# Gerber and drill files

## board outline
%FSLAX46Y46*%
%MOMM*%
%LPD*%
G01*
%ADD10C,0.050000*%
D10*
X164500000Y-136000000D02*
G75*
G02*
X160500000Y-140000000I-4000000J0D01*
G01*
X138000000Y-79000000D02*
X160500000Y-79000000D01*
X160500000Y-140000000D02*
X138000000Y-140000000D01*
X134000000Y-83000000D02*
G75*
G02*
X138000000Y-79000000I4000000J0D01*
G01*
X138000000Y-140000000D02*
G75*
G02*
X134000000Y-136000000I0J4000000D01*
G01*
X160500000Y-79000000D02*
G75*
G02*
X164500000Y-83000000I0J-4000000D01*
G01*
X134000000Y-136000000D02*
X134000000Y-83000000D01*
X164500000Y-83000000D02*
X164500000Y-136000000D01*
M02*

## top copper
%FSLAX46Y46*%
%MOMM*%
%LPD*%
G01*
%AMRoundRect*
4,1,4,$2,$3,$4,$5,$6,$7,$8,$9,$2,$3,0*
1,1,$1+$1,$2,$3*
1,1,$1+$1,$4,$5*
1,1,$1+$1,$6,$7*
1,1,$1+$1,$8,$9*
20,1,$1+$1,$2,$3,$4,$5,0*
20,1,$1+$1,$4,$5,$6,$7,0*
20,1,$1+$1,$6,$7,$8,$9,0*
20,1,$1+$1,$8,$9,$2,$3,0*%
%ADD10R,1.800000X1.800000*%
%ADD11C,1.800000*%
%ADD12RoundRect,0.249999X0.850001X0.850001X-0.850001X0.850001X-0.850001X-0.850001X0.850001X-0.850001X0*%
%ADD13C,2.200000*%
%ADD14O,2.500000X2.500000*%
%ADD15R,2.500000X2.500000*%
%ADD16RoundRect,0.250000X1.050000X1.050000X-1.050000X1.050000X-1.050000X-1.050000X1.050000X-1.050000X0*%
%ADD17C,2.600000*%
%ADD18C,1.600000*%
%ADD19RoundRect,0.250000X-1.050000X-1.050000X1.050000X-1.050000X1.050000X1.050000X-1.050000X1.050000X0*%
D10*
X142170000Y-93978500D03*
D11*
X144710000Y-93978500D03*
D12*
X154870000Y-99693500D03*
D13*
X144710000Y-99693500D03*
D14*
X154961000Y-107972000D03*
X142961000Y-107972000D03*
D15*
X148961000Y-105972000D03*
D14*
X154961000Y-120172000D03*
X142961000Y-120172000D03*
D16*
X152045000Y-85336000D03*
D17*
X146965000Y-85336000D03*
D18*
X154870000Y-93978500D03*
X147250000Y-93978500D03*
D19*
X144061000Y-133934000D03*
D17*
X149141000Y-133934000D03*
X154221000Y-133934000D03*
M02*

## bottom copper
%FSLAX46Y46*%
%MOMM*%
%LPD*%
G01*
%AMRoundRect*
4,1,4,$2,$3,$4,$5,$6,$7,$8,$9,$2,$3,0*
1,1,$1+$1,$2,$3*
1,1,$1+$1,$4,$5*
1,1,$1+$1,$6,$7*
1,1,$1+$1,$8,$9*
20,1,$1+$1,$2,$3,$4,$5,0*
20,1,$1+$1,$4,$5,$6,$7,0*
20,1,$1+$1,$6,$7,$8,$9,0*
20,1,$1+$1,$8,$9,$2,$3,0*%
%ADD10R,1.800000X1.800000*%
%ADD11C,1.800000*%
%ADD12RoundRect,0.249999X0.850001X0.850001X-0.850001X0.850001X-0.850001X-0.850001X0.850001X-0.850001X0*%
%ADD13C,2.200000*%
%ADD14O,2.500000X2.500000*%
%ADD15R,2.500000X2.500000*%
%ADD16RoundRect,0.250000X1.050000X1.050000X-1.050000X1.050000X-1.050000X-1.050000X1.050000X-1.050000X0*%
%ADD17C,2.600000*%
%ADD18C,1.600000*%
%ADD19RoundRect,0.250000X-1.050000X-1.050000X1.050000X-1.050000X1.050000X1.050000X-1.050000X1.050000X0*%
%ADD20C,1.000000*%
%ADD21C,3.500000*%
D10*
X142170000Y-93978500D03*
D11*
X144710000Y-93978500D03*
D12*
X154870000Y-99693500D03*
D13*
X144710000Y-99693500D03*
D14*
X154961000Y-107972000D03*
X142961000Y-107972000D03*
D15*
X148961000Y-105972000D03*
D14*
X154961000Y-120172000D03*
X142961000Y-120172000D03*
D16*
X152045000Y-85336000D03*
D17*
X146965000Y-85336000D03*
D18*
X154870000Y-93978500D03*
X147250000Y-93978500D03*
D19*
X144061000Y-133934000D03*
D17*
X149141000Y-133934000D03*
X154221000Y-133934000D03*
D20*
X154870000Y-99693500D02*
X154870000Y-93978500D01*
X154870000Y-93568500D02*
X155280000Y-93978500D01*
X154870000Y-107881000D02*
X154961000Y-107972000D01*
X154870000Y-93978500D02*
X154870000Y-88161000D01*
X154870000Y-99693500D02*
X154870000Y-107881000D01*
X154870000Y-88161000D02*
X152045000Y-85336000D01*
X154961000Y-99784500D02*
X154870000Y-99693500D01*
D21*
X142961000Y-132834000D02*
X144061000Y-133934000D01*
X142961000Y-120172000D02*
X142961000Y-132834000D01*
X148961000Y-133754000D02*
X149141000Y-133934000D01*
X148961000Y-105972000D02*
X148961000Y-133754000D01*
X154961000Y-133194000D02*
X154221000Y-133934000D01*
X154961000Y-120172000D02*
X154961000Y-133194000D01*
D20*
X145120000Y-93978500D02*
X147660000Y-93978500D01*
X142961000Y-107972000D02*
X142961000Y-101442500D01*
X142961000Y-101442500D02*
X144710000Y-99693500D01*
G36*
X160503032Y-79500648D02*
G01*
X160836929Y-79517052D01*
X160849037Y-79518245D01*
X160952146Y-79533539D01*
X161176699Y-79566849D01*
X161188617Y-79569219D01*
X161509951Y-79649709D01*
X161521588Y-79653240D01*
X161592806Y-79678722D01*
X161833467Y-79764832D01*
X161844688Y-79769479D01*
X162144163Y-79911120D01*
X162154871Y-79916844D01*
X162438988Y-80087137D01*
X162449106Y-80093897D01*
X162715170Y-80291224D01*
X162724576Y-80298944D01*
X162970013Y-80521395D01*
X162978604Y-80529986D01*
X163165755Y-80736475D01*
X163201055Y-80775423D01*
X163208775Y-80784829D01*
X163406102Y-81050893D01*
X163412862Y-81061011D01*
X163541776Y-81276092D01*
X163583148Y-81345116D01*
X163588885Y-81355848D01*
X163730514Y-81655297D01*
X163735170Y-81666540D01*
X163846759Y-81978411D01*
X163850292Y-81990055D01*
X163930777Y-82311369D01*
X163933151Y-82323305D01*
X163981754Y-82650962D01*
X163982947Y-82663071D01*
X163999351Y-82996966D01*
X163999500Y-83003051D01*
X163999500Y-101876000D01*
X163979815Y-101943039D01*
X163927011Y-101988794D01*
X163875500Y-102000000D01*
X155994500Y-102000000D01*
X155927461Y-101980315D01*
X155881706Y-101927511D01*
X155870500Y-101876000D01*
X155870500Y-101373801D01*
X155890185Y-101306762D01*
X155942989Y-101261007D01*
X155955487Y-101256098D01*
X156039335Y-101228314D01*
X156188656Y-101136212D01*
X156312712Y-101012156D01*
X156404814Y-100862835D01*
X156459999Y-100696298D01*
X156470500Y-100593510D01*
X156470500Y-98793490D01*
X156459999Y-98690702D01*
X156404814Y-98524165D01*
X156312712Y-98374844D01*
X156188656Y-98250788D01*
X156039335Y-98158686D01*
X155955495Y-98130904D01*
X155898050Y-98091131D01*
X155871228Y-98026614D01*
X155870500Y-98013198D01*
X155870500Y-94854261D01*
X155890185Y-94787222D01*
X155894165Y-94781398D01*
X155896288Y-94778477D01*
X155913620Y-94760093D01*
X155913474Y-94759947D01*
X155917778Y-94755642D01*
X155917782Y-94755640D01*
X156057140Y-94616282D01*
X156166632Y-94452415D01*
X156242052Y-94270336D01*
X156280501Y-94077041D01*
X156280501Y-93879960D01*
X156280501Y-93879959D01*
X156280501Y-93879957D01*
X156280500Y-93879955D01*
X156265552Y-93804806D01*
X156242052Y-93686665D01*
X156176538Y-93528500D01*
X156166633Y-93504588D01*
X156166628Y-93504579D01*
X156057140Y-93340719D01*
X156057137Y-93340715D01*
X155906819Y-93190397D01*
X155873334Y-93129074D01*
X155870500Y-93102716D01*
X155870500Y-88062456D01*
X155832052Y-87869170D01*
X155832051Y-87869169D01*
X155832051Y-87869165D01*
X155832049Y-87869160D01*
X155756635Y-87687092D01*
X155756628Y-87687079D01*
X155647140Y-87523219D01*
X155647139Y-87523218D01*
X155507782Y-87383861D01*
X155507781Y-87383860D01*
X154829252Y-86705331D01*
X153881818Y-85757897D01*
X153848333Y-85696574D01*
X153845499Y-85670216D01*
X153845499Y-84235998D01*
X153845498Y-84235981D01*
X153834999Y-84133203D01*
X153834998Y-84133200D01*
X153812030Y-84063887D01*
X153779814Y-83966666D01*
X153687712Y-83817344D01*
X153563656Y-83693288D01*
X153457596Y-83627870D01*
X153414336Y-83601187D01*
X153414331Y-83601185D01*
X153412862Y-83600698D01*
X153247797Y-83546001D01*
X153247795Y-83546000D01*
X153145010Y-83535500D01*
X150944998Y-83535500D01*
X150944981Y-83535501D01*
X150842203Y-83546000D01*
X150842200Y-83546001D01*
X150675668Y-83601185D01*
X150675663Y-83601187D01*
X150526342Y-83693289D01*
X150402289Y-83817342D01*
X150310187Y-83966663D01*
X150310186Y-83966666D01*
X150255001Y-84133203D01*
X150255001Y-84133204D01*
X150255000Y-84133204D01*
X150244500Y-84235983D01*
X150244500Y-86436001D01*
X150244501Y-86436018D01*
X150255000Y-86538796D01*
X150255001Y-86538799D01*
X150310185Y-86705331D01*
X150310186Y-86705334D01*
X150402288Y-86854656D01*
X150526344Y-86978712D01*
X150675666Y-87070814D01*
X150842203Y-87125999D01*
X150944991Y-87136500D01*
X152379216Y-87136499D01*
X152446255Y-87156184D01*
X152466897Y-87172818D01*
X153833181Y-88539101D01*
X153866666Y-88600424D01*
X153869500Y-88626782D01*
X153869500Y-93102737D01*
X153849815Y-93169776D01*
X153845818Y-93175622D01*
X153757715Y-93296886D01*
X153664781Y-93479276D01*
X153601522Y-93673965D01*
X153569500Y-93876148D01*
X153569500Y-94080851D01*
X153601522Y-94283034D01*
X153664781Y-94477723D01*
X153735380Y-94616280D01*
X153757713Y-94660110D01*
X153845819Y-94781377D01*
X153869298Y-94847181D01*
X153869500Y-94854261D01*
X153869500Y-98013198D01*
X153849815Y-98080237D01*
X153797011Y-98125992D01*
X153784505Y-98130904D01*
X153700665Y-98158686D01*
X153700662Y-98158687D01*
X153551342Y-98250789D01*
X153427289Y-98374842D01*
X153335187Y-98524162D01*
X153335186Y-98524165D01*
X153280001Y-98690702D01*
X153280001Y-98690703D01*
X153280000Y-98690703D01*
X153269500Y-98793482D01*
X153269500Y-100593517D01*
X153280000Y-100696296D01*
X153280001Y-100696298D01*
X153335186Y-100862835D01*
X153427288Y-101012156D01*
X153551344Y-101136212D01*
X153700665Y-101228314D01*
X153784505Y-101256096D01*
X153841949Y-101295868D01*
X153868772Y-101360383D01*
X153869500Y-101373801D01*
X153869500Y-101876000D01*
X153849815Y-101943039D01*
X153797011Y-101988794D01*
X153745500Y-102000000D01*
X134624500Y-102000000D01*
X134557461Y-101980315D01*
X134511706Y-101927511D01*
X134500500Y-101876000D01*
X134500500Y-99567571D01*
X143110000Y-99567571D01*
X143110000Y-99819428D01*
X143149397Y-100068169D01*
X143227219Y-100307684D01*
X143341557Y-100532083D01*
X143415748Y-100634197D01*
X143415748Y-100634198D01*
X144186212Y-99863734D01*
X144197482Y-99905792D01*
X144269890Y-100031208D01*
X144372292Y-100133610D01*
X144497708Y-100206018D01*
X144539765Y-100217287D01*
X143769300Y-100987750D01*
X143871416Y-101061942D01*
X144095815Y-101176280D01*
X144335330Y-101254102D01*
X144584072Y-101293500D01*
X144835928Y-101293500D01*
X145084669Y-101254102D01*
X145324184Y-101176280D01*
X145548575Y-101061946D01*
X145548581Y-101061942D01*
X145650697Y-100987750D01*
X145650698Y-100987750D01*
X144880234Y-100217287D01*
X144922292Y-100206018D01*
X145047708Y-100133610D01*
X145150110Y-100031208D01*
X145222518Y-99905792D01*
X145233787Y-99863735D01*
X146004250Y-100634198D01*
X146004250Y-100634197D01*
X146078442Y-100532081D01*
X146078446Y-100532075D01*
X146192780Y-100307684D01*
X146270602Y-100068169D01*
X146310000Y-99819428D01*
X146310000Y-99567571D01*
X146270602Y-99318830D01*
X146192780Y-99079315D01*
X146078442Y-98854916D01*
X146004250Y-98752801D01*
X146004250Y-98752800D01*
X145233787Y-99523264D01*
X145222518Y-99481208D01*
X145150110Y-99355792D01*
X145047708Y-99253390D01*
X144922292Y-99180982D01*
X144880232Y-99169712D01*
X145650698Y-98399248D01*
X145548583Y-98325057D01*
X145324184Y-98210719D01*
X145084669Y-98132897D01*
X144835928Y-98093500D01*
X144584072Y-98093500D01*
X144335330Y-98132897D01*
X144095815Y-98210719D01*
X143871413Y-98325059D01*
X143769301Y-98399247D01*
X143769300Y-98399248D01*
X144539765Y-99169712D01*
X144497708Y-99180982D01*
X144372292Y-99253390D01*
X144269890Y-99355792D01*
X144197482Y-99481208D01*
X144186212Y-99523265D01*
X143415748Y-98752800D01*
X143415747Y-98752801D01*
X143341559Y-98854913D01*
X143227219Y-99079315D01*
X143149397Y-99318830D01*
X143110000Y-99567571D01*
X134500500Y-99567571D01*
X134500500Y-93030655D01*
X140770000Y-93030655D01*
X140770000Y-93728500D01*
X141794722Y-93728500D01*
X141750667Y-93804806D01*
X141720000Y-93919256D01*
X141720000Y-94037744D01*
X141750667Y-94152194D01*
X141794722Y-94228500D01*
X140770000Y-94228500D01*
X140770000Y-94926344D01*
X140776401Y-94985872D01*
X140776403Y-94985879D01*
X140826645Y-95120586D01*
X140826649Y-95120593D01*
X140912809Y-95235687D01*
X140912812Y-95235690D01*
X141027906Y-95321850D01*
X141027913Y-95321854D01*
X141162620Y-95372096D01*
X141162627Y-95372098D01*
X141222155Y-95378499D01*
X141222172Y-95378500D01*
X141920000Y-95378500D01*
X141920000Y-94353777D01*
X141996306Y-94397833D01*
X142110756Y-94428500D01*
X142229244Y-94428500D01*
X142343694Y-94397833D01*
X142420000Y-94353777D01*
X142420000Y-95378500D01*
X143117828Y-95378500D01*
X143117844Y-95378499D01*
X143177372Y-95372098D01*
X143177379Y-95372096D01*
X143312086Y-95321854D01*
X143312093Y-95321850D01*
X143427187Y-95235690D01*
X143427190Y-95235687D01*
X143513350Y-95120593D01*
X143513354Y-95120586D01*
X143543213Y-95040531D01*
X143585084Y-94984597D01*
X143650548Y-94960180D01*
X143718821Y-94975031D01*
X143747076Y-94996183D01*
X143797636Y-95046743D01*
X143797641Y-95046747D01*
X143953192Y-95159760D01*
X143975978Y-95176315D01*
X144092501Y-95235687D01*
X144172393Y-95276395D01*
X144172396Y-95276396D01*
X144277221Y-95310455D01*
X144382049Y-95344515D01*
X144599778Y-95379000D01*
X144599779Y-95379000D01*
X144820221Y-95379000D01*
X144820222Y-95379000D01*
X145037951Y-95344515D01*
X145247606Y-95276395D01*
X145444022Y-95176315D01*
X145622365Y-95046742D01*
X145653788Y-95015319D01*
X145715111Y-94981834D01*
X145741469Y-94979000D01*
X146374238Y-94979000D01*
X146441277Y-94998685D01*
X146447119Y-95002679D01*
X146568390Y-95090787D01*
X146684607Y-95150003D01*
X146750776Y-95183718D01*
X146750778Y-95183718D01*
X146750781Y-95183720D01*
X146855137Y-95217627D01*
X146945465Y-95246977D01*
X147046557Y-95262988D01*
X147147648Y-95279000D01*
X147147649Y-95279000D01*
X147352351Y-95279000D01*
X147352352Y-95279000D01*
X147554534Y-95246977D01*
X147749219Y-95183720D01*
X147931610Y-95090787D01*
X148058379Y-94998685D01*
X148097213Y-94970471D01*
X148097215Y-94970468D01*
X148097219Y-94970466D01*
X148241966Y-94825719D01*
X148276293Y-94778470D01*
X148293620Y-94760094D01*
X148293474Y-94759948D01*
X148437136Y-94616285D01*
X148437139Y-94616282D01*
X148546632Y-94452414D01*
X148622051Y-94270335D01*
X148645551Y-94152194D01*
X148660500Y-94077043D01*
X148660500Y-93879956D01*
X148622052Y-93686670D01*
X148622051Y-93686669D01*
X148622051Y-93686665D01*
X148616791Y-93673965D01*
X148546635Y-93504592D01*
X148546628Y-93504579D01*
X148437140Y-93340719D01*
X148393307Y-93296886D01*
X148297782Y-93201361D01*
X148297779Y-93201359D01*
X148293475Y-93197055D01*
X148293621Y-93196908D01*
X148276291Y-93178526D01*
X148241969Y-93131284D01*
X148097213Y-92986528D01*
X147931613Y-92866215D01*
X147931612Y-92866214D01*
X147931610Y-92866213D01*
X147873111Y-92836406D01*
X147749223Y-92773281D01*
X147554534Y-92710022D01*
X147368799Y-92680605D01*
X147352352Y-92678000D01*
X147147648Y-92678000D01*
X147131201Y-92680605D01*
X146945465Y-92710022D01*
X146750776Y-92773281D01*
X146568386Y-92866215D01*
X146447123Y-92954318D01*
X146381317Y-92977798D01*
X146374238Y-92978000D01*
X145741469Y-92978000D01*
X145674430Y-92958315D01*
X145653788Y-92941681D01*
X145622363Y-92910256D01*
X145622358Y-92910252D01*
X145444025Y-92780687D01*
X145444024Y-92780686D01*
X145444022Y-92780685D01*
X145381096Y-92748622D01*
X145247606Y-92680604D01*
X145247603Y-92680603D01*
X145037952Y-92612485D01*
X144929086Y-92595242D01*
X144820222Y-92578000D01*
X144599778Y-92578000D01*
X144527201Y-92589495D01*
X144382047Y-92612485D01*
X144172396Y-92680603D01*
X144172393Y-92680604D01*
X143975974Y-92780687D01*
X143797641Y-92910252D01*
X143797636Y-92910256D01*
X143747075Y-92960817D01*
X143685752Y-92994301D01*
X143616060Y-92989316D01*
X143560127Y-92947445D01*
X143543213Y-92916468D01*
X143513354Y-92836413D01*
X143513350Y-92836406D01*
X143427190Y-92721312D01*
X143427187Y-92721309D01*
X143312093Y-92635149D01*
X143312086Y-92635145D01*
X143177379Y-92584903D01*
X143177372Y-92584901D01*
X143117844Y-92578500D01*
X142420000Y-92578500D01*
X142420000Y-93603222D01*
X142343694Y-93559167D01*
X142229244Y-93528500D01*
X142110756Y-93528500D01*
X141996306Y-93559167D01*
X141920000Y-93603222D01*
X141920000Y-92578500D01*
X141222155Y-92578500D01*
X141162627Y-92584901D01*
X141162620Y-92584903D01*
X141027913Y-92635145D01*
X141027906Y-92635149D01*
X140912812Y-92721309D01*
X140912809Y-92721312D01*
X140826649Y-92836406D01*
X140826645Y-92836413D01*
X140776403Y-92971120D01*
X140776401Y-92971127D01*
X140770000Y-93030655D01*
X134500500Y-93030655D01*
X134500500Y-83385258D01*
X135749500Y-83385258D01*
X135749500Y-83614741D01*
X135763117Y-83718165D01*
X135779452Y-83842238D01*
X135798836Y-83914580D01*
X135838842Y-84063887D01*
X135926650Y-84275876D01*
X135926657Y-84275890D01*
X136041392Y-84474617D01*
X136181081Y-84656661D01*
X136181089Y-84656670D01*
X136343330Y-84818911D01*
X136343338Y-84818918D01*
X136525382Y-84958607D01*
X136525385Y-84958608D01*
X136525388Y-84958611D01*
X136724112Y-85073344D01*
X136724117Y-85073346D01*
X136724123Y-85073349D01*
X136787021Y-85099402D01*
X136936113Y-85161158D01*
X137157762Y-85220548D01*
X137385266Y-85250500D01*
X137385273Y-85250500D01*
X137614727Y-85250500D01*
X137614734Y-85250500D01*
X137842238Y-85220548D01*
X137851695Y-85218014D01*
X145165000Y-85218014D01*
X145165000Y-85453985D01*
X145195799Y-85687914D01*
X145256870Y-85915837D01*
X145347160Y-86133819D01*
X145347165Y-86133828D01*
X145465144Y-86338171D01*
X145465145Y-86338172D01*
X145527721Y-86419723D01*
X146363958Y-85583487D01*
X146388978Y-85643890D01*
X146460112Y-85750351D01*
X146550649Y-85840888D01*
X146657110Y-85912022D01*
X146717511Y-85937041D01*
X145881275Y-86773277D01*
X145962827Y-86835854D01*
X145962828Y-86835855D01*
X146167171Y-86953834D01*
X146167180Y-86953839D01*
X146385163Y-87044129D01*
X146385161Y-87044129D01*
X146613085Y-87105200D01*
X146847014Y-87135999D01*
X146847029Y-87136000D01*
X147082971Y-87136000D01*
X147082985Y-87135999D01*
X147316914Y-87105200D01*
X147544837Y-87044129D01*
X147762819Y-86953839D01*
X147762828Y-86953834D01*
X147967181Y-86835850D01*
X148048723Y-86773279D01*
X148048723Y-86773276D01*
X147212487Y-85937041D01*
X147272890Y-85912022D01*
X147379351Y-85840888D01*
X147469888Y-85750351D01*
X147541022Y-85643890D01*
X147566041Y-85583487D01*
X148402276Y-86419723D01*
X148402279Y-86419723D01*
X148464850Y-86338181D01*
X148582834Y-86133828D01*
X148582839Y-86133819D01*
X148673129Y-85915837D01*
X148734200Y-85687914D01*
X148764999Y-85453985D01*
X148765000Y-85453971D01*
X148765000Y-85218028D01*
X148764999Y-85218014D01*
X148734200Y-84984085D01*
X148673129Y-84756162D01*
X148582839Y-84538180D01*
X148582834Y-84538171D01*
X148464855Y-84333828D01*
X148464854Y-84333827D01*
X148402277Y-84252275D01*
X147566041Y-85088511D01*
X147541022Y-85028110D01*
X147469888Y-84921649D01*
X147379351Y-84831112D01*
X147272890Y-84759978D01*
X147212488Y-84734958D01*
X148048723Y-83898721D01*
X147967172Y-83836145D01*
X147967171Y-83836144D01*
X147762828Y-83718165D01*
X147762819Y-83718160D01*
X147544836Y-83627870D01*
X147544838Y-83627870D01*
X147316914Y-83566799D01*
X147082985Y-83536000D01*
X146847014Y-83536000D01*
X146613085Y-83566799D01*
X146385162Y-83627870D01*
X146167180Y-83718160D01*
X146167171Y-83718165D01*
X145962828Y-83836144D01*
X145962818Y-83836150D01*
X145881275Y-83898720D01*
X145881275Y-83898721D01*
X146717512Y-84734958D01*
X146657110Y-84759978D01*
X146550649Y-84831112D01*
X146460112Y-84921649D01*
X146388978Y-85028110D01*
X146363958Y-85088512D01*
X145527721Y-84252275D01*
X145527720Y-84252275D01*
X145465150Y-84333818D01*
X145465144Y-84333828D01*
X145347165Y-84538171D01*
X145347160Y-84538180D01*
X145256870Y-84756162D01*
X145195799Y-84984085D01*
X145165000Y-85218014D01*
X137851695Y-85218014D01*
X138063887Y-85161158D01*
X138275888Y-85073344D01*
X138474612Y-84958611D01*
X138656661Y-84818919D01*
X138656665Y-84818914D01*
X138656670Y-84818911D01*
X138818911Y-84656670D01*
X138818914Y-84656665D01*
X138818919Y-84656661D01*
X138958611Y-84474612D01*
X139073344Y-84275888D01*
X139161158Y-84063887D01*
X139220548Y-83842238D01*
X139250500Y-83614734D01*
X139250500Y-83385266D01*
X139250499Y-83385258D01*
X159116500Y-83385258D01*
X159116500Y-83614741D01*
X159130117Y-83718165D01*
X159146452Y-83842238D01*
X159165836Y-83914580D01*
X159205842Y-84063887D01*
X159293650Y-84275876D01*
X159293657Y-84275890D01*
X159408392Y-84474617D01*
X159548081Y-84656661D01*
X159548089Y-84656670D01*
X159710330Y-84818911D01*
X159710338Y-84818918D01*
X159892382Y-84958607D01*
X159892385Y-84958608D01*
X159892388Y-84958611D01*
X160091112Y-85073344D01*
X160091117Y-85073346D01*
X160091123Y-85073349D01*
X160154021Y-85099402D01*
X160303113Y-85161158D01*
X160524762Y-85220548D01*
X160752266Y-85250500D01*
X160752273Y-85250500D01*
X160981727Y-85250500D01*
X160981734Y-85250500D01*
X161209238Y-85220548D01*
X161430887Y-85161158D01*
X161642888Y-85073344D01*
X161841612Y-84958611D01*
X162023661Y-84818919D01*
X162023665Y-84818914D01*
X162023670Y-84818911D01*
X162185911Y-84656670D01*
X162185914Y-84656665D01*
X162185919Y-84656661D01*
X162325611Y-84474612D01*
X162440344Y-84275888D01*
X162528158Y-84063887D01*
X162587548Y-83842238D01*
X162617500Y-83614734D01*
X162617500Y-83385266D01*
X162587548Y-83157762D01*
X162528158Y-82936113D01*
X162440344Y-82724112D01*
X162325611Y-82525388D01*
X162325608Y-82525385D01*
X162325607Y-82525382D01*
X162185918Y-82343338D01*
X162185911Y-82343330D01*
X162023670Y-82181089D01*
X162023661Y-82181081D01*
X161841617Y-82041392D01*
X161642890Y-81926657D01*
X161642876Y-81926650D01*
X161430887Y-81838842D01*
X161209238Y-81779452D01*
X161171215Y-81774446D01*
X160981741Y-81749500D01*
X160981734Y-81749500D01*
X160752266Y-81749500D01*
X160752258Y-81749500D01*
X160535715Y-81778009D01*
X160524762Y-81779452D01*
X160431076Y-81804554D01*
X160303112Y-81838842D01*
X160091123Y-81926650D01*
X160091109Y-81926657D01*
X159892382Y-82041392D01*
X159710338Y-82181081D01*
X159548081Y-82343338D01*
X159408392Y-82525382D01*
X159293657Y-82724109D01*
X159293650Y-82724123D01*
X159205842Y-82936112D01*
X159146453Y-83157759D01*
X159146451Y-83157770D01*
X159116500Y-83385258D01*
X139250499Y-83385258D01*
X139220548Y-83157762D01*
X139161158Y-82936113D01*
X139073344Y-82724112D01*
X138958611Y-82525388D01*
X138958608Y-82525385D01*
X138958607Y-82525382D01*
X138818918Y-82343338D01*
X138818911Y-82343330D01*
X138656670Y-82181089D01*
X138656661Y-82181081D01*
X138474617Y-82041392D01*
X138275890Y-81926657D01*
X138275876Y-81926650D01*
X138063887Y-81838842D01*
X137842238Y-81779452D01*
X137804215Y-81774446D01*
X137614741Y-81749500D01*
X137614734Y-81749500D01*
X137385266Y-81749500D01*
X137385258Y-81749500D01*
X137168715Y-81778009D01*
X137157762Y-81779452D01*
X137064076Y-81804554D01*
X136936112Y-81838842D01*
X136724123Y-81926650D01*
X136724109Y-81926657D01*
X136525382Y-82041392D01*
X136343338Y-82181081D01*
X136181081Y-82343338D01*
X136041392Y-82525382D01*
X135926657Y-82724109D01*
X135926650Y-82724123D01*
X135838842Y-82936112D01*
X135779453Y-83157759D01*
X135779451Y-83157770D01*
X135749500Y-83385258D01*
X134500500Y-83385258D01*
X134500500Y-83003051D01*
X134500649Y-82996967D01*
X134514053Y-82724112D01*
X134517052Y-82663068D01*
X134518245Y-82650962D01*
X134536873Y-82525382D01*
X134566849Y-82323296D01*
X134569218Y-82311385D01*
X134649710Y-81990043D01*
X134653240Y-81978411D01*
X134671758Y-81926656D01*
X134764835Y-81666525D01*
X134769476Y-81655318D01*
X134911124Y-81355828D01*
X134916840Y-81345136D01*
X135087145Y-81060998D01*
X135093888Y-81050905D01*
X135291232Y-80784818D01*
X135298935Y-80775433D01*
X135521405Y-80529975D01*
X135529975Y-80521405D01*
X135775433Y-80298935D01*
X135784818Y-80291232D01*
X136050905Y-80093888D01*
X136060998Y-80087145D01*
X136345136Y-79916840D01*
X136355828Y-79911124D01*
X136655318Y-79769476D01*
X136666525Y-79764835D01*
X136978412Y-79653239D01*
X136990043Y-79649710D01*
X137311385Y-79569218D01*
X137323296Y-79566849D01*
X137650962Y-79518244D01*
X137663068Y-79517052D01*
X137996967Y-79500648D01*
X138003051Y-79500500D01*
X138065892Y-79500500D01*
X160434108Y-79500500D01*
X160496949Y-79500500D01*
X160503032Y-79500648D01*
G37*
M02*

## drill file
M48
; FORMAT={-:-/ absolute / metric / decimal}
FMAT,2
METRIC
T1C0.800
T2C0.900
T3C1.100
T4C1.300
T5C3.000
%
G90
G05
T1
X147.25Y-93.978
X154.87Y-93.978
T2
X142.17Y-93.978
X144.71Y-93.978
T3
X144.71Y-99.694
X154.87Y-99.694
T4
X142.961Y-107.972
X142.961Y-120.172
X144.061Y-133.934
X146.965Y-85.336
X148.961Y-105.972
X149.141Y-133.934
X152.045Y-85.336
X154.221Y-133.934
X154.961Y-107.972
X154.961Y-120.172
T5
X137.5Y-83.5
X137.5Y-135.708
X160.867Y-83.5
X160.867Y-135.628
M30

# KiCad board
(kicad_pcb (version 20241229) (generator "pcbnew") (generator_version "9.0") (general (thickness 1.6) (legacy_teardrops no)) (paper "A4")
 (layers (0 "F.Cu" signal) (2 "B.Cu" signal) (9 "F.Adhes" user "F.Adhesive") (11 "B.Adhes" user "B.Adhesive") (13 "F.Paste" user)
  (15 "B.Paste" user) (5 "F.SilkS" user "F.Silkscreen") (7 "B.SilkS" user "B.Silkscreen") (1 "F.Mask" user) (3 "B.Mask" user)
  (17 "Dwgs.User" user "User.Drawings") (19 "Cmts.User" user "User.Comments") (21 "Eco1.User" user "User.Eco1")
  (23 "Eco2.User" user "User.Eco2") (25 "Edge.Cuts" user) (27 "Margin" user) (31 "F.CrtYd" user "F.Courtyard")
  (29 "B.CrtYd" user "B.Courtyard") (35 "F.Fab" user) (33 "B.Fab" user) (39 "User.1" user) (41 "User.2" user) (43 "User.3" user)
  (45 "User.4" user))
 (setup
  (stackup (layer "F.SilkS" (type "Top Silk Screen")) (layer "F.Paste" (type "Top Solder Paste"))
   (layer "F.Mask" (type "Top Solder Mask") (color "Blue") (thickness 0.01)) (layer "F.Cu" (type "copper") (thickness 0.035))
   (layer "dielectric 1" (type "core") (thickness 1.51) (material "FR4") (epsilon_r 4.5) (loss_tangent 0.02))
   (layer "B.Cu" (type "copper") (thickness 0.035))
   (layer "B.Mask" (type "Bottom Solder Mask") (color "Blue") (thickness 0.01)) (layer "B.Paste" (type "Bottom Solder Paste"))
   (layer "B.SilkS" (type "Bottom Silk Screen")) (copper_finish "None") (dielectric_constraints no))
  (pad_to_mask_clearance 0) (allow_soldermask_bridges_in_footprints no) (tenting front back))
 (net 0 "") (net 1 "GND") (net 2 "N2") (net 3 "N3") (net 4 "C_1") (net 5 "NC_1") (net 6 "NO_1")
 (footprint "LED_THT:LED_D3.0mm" (layer "F.Cu") (at 142.17 93.9785)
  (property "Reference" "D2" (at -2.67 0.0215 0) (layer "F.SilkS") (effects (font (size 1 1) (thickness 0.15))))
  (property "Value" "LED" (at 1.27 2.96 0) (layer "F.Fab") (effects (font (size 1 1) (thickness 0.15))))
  (pad "1" thru_hole rect (at 0 0) (size 1.8 1.8) (drill 0.9) (layers "*.Cu" "*.Mask") (remove_unused_layers no) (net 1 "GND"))
  (pad "2" thru_hole circle (at 2.54 0) (size 1.8 1.8) (drill 0.9) (layers "*.Cu" "*.Mask") (remove_unused_layers no) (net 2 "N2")))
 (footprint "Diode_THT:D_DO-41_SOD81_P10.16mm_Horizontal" (layer "F.Cu") (at 154.87 99.6935 180)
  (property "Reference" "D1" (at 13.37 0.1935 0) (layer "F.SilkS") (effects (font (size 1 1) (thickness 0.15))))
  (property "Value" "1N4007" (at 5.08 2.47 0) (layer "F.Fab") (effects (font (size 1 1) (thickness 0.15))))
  (pad "1" thru_hole roundrect (at 0 0 180) (size 2.2 2.2) (drill 1.1) (layers "*.Cu" "*.Mask") (remove_unused_layers no)
   (roundrect_rratio 0.113636) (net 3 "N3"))
  (pad "2" thru_hole circle (at 10.16 0 180) (size 2.2 2.2) (drill 1.1) (layers "*.Cu" "*.Mask") (remove_unused_layers no) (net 1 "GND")))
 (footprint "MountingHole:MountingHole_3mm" (layer "F.Cu") (at 160.867 83.5 90)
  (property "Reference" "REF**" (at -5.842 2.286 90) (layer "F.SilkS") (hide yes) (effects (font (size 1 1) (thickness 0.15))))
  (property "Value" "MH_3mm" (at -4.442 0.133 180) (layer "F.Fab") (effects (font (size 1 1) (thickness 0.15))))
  (pad "" np_thru_hole circle (at 0 0 90) (size 3 3) (drill 3) (layers "*.Cu" "*.Mask")))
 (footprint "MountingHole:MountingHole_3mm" (layer "F.Cu") (at 137.5 135.708 90)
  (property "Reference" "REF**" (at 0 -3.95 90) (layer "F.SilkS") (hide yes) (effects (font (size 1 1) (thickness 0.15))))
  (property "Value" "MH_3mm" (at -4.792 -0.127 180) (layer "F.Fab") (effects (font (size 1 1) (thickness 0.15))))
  (pad "" np_thru_hole circle (at 0 0 90) (size 3 3) (drill 3) (layers "*.Cu" "*.Mask")))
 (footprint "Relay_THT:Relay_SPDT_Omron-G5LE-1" (layer "F.Cu") (at 148.961 105.972)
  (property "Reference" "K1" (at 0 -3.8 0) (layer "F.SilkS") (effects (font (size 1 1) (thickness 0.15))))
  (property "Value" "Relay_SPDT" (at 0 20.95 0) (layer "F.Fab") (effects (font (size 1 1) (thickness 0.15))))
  (pad "1" thru_hole oval (at 6 2) (size 2.5 2.5) (drill 1.3) (layers "*.Cu" "*.Mask") (remove_unused_layers no) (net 3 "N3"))
  (pad "2" thru_hole oval (at -6 2) (size 2.5 2.5) (drill 1.3) (layers "*.Cu" "*.Mask") (remove_unused_layers no) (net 1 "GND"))
  (pad "3" thru_hole rect (at 0 0) (size 2.5 2.5) (drill 1.3) (layers "*.Cu" "*.Mask") (remove_unused_layers no) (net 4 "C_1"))
  (pad "4" thru_hole oval (at 6 14.2) (size 2.5 2.5) (drill 1.3) (layers "*.Cu" "*.Mask") (remove_unused_layers no) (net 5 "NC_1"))
  (pad "5" thru_hole oval (at -6 14.2) (size 2.5 2.5) (drill 1.3) (layers "*.Cu" "*.Mask") (remove_unused_layers no) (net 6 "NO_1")))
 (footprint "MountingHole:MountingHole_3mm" (layer "F.Cu") (at 137.5 83.5 90)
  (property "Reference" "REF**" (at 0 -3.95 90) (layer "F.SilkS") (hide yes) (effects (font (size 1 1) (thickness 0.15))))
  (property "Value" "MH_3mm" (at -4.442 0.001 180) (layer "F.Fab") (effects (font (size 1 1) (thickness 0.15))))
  (pad "" np_thru_hole circle (at 0 0 90) (size 3 3) (drill 3) (layers "*.Cu" "*.Mask")))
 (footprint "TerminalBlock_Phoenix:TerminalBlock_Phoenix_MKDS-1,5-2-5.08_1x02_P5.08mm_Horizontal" (layer "F.Cu") (at 152.045 85.336 180)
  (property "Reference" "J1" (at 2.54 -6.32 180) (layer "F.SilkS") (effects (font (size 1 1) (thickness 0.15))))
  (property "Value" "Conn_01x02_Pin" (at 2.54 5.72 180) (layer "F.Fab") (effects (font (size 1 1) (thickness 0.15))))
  (pad "1" thru_hole roundrect (at 0 0 180) (size 2.6 2.6) (drill 1.3) (layers "*.Cu" "*.Mask") (remove_unused_layers no)
   (roundrect_rratio 0.096154) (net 3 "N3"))
  (pad "2" thru_hole circle (at 5.08 0 180) (size 2.6 2.6) (drill 1.3) (layers "*.Cu" "*.Mask") (remove_unused_layers no) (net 1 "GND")))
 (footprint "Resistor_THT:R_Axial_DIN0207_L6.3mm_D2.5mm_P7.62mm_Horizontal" (layer "F.Cu") (at 154.87 93.9785 180)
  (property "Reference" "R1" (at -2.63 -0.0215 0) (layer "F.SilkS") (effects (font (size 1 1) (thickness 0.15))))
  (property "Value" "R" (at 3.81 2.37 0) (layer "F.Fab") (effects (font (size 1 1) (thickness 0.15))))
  (pad "1" thru_hole circle (at 0 0 180) (size 1.6 1.6) (drill 0.8) (layers "*.Cu" "*.Mask") (remove_unused_layers no) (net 3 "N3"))
  (pad "2" thru_hole circle (at 7.62 0 180) (size 1.6 1.6) (drill 0.8) (layers "*.Cu" "*.Mask") (remove_unused_layers no) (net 2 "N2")))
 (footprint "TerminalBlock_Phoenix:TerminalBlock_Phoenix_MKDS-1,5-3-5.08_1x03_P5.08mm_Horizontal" (layer "F.Cu") (at 144.061 133.934)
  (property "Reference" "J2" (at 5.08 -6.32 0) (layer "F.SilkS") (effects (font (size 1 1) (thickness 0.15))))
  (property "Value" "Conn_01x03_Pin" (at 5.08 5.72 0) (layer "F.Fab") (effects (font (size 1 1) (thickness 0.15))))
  (pad "1" thru_hole roundrect (at 0 0) (size 2.6 2.6) (drill 1.3) (layers "*.Cu" "*.Mask") (remove_unused_layers no)
   (roundrect_rratio 0.096154) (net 6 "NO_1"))
  (pad "2" thru_hole circle (at 5.08 0) (size 2.6 2.6) (drill 1.3) (layers "*.Cu" "*.Mask") (remove_unused_layers no) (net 4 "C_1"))
  (pad "3" thru_hole circle (at 10.16 0) (size 2.6 2.6) (drill 1.3) (layers "*.Cu" "*.Mask") (remove_unused_layers no) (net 5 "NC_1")))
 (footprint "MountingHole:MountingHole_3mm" (layer "F.Cu") (at 160.867 135.628 90)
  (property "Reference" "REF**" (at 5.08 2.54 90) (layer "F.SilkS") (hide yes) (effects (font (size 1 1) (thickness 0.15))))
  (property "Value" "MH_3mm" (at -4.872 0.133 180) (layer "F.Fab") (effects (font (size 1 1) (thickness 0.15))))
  (pad "" np_thru_hole circle (at 0 0 90) (size 3 3) (drill 3) (layers "*.Cu" "*.Mask")))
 (gr_arc (start 164.5 136) (mid 163.328427 138.828427) (end 160.5 140) (stroke (width 0.05) (type default)) (layer "Edge.Cuts"))
 (gr_line (start 138 79) (end 160.5 79) (stroke (width 0.05) (type default)) (layer "Edge.Cuts"))
 (gr_line (start 160.5 140) (end 138 140) (stroke (width 0.05) (type default)) (layer "Edge.Cuts"))
 (gr_arc (start 134 83) (mid 135.171573 80.171573) (end 138 79) (stroke (width 0.05) (type default)) (layer "Edge.Cuts"))
 (gr_arc (start 138 140) (mid 135.171573 138.828427) (end 134 136) (stroke (width 0.05) (type default)) (layer "Edge.Cuts"))
 (gr_arc (start 160.5 79) (mid 163.328427 80.171573) (end 164.5 83) (stroke (width 0.05) (type default)) (layer "Edge.Cuts"))
 (gr_line (start 134 136) (end 134 83) (stroke (width 0.05) (type default)) (layer "Edge.Cuts"))
 (gr_line (start 164.5 83) (end 164.5 136) (stroke (width 0.05) (type default)) (layer "Edge.Cuts"))
 (segment (start 154.87 99.6935) (end 154.87 93.9785) (width 1) (layer "B.Cu") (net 3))
 (segment (start 154.87 93.5685) (end 155.28 93.9785) (width 1) (layer "B.Cu") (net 3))
 (segment (start 154.87 107.881) (end 154.961 107.972) (width 1) (layer "B.Cu") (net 3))
 (segment (start 154.87 93.9785) (end 154.87 88.161) (width 1) (layer "B.Cu") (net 3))
 (segment (start 154.87 99.6935) (end 154.87 107.881) (width 1) (layer "B.Cu") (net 3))
 (segment (start 154.87 88.161) (end 152.045 85.336) (width 1) (layer "B.Cu") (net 3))
 (segment (start 154.961 99.7845) (end 154.87 99.6935) (width 1) (layer "B.Cu") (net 3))
 (segment (start 142.961 132.834) (end 144.061 133.934) (width 3.5) (layer "B.Cu") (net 6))
 (segment (start 142.961 120.172) (end 142.961 132.834) (width 3.5) (layer "B.Cu") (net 6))
 (segment (start 148.961 133.754) (end 149.141 133.934) (width 3.5) (layer "B.Cu") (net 4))
 (segment (start 148.961 105.972) (end 148.961 133.754) (width 3.5) (layer "B.Cu") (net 4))
 (segment (start 154.961 133.194) (end 154.221 133.934) (width 3.5) (layer "B.Cu") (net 5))
 (segment (start 154.961 120.172) (end 154.961 133.194) (width 3.5) (layer "B.Cu") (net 5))
 (segment (start 145.12 93.9785) (end 147.66 93.9785) (width 1) (layer "B.Cu") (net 2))
 (segment (start 142.961 107.972) (end 142.961 101.4425) (width 1) (layer "B.Cu") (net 1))
 (segment (start 142.961 101.4425) (end 144.71 99.6935) (width 1) (layer "B.Cu") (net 1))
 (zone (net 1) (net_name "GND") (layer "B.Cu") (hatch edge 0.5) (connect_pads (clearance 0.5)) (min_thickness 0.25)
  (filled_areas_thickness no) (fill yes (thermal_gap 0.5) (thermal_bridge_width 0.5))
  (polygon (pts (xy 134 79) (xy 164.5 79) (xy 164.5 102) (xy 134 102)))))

